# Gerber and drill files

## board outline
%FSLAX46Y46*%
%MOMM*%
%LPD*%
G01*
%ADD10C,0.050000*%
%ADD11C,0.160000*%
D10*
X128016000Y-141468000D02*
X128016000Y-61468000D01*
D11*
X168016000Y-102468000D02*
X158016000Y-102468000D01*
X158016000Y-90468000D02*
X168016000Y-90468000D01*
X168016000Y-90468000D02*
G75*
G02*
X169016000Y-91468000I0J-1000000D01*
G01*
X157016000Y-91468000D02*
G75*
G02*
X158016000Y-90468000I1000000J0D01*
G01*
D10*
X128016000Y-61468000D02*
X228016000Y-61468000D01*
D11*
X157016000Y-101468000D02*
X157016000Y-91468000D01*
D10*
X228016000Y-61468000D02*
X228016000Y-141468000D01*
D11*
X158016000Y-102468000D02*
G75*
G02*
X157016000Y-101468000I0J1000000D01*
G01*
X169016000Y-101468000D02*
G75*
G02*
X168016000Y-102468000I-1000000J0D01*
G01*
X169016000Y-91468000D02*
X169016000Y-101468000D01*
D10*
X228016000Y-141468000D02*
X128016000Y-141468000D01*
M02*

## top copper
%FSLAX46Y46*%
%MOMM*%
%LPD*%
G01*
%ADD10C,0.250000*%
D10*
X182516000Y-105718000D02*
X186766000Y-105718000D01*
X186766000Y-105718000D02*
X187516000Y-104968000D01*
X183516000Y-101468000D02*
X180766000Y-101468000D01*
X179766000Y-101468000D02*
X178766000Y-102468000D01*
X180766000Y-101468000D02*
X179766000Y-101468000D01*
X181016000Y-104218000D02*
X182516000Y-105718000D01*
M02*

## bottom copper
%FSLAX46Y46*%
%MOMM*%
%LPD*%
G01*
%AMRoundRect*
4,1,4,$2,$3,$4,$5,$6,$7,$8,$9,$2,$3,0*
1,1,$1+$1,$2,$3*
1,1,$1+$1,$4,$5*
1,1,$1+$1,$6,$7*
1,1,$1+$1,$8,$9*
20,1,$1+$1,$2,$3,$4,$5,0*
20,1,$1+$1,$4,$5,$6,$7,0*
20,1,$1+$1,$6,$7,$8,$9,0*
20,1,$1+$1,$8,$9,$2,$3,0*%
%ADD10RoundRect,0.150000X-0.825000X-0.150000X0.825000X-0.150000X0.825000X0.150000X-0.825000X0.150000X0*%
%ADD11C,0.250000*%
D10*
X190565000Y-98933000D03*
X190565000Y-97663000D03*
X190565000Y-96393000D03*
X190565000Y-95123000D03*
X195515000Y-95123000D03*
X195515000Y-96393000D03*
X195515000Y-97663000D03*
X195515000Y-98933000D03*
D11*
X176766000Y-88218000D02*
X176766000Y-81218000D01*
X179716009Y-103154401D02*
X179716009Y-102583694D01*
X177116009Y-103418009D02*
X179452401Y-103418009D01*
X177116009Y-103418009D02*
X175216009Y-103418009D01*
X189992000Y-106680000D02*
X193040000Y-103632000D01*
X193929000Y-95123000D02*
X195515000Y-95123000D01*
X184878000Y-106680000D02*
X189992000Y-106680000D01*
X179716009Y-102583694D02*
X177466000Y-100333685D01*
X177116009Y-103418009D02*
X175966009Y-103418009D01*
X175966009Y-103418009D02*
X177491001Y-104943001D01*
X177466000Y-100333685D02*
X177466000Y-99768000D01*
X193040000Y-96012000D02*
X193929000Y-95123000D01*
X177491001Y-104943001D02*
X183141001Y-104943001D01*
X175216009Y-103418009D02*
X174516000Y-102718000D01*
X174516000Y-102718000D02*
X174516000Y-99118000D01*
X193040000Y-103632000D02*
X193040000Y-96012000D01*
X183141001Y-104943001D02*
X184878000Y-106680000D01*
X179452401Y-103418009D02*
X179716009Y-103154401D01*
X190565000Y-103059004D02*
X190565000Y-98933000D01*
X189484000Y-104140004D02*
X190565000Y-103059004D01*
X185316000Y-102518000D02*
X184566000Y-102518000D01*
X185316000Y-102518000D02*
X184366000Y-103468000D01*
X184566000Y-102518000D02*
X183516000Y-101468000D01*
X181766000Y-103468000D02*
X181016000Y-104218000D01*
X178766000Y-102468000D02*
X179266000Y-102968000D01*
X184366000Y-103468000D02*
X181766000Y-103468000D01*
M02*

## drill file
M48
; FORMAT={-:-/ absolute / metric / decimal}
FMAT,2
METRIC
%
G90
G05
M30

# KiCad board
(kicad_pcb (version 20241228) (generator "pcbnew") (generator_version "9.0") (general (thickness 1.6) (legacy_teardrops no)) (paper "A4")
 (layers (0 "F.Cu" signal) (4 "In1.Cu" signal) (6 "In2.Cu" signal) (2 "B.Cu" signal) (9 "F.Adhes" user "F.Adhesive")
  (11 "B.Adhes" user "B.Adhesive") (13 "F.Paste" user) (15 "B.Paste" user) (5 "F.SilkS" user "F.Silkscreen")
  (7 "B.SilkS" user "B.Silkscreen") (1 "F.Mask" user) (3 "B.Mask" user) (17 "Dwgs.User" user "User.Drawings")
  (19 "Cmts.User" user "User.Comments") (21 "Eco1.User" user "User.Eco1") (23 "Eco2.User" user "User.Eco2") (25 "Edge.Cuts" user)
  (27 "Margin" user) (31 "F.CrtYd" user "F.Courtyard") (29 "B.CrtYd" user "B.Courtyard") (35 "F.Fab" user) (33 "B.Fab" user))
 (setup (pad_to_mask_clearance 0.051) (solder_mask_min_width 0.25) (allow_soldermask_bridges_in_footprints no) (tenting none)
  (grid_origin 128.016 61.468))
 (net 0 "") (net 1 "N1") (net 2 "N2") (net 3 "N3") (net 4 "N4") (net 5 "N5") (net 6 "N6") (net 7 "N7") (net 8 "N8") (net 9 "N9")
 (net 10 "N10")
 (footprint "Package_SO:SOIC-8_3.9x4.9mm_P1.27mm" (layer "B.Cu") (at 193.04 97.028)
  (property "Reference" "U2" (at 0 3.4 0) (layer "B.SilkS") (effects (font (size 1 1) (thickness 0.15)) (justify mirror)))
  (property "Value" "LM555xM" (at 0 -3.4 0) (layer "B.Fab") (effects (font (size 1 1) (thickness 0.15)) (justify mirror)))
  (pad "1" smd roundrect (at -2.475 1.905) (size 1.95 0.6) (layers "B.Cu" "B.Mask" "B.Paste") (roundrect_rratio 0.25) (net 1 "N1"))
  (pad "2" smd roundrect (at -2.475 0.635) (size 1.95 0.6) (layers "B.Cu" "B.Mask" "B.Paste") (roundrect_rratio 0.25) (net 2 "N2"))
  (pad "3" smd roundrect (at -2.475 -0.635) (size 1.95 0.6) (layers "B.Cu" "B.Mask" "B.Paste") (roundrect_rratio 0.25) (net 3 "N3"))
  (pad "4" smd roundrect (at -2.475 -1.905) (size 1.95 0.6) (layers "B.Cu" "B.Mask" "B.Paste") (roundrect_rratio 0.25) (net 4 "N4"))
  (pad "5" smd roundrect (at 2.475 -1.905) (size 1.95 0.6) (layers "B.Cu" "B.Mask" "B.Paste") (roundrect_rratio 0.25) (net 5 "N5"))
  (pad "6" smd roundrect (at 2.475 -0.635) (size 1.95 0.6) (layers "B.Cu" "B.Mask" "B.Paste") (roundrect_rratio 0.25) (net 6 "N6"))
  (pad "7" smd roundrect (at 2.475 0.635) (size 1.95 0.6) (layers "B.Cu" "B.Mask" "B.Paste") (roundrect_rratio 0.25) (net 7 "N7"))
  (pad "8" smd roundrect (at 2.475 1.905) (size 1.95 0.6) (layers "B.Cu" "B.Mask" "B.Paste") (roundrect_rratio 0.25) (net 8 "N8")))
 (gr_line (start 128.016 141.468) (end 128.016 61.468) (stroke (width 0.05) (type solid)) (layer "Edge.Cuts"))
 (gr_line (start 168.016 102.468) (end 158.016 102.468) (stroke (width 0.16) (type solid)) (layer "Edge.Cuts"))
 (gr_line (start 158.016 90.468) (end 168.016 90.468) (stroke (width 0.16) (type solid)) (layer "Edge.Cuts"))
 (gr_arc (start 168.016 90.468) (mid 168.723107 90.760893) (end 169.016 91.468) (stroke (width 0.16) (type solid)) (layer "Edge.Cuts"))
 (gr_arc (start 157.016 91.468) (mid 157.308893 90.760893) (end 158.016 90.468) (stroke (width 0.16) (type solid)) (layer "Edge.Cuts"))
 (gr_line (start 128.016 61.468) (end 228.016 61.468) (stroke (width 0.05) (type solid)) (layer "Edge.Cuts"))
 (gr_line (start 157.016 101.468) (end 157.016 91.468) (stroke (width 0.16) (type solid)) (layer "Edge.Cuts"))
 (gr_line (start 228.016 61.468) (end 228.016 141.468) (stroke (width 0.05) (type solid)) (layer "Edge.Cuts"))
 (gr_arc (start 158.016 102.468) (mid 157.308893 102.175107) (end 157.016 101.468) (stroke (width 0.16) (type solid)) (layer "Edge.Cuts"))
 (gr_arc (start 169.016 101.468) (mid 168.723107 102.175107) (end 168.016 102.468) (stroke (width 0.16) (type solid)) (layer "Edge.Cuts"))
 (gr_line (start 169.016 91.468) (end 169.016 101.468) (stroke (width 0.16) (type solid)) (layer "Edge.Cuts"))
 (gr_line (start 228.016 141.468) (end 128.016 141.468) (stroke (width 0.05) (type solid)) (layer "Edge.Cuts"))
 (segment (start 176.766 88.218) (end 176.766 81.218) (width 0.25) (layer "B.Cu") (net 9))
 (segment (start 179.716009 103.154401) (end 179.716009 102.583694) (width 0.25) (layer "B.Cu") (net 5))
 (segment (start 177.116009 103.418009) (end 179.452401 103.418009) (width 0.25) (layer "B.Cu") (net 5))
 (segment (start 177.116009 103.418009) (end 175.216009 103.418009) (width 0.25) (layer "B.Cu") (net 5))
 (segment (start 189.992 106.68) (end 193.04 103.632) (width 0.25) (layer "B.Cu") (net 5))
 (segment (start 193.929 95.123) (end 195.515 95.123) (width 0.25) (layer "B.Cu") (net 5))
 (segment (start 184.878 106.68) (end 189.992 106.68) (width 0.25) (layer "B.Cu") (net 5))
 (segment (start 179.716009 102.583694) (end 177.466 100.333685) (width 0.25) (layer "B.Cu") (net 5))
 (segment (start 177.116009 103.418009) (end 175.966009 103.418009) (width 0.25) (layer "B.Cu") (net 5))
 (segment (start 175.966009 103.418009) (end 177.491001 104.943001) (width 0.25) (layer "B.Cu") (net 5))
 (segment (start 177.466 100.333685) (end 177.466 99.768) (width 0.25) (layer "B.Cu") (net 5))
 (segment (start 193.04 96.012) (end 193.929 95.123) (width 0.25) (layer "B.Cu") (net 5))
 (segment (start 177.491001 104.943001) (end 183.141001 104.943001) (width 0.25) (layer "B.Cu") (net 5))
 (segment (start 175.216009 103.418009) (end 174.516 102.718) (width 0.25) (layer "B.Cu") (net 5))
 (segment (start 174.516 102.718) (end 174.516 99.118) (width 0.25) (layer "B.Cu") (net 5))
 (segment (start 193.04 103.632) (end 193.04 96.012) (width 0.25) (layer "B.Cu") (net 5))
 (segment (start 183.141001 104.943001) (end 184.878 106.68) (width 0.25) (layer "B.Cu") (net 5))
 (segment (start 179.452401 103.418009) (end 179.716009 103.154401) (width 0.25) (layer "B.Cu") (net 5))
 (segment (start 190.565 103.059004) (end 190.565 98.933) (width 0.25) (layer "B.Cu") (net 1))
 (segment (start 189.484 104.140004) (end 190.565 103.059004) (width 0.25) (layer "B.Cu") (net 1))
 (segment (start 182.516 105.718) (end 186.766 105.718) (width 0.25) (layer "F.Cu") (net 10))
 (segment (start 186.766 105.718) (end 187.516 104.968) (width 0.25) (layer "F.Cu") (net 10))
 (segment (start 183.516 101.468) (end 180.766 101.468) (width 0.25) (layer "F.Cu") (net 10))
 (segment (start 179.766 101.468) (end 178.766 102.468) (width 0.25) (layer "F.Cu") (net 10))
 (segment (start 180.766 101.468) (end 179.766 101.468) (width 0.25) (layer "F.Cu") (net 10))
 (segment (start 181.016 104.218) (end 182.516 105.718) (width 0.25) (layer "F.Cu") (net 10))
 (segment (start 185.316 102.518) (end 184.566 102.518) (width 0.25) (layer "B.Cu") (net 10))
 (segment (start 185.316 102.518) (end 184.366 103.468) (width 0.25) (layer "B.Cu") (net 10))
 (segment (start 184.566 102.518) (end 183.516 101.468) (width 0.25) (layer "B.Cu") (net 10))
 (segment (start 181.766 103.468) (end 181.016 104.218) (width 0.25) (layer "B.Cu") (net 10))
 (segment (start 178.766 102.468) (end 179.266 102.968) (width 0.25) (layer "B.Cu") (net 10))
 (segment (start 184.366 103.468) (end 181.766 103.468) (width 0.25) (layer "B.Cu") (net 10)))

